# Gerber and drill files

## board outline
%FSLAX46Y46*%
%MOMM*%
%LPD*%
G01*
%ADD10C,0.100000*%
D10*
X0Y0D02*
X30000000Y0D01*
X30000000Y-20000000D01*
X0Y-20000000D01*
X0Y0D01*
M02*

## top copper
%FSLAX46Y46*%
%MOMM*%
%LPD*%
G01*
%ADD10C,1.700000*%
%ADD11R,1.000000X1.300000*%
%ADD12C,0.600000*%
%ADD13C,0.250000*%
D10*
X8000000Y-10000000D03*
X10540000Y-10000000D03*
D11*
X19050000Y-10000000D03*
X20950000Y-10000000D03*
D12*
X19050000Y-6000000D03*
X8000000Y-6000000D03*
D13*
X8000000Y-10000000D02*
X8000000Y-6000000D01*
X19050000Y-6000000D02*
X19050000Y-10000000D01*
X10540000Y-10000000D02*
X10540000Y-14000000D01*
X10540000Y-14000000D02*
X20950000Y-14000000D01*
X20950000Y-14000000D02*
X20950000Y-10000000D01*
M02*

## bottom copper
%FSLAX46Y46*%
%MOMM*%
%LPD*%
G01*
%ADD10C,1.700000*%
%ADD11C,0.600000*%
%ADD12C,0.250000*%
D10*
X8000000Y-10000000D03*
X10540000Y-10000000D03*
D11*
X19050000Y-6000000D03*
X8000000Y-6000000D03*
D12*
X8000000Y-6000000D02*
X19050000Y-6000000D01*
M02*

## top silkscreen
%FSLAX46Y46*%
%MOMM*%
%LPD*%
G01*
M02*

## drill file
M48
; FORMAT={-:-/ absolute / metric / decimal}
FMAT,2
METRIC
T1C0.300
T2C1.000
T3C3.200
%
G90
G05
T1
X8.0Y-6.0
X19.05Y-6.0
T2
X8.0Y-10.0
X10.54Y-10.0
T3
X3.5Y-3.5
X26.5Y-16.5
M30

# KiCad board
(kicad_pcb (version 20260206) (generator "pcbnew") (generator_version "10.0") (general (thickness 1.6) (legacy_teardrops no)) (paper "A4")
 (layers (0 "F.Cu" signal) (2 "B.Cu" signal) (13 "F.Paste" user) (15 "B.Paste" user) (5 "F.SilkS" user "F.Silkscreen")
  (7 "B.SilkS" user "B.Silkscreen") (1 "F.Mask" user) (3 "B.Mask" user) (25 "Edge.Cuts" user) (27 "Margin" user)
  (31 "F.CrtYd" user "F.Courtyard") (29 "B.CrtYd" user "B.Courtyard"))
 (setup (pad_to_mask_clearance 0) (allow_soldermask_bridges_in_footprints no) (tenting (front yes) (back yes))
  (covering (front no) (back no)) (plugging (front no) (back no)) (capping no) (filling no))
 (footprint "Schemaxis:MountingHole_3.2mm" (layer "F.Cu") (at 26.5 16.5)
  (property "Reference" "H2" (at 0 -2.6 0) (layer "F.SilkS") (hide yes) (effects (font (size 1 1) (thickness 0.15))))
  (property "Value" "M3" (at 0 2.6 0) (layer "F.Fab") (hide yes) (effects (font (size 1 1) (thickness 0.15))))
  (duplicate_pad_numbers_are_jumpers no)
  (pad "" np_thru_hole circle (at 0 0) (size 3.2 3.2) (drill 3.2) (layers "*.Cu" "*.Mask")))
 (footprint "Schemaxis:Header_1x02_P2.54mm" (layer "F.Cu") (at 8 10 90)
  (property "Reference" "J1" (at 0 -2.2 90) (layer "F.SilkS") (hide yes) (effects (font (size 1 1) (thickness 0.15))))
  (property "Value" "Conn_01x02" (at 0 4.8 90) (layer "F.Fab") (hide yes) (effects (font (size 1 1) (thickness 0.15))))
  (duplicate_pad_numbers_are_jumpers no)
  (pad "1" thru_hole circle (at 0 0 90) (size 1.7 1.7) (drill 1) (layers "*.Cu" "*.Mask") (remove_unused_layers no) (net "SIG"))
  (pad "2" thru_hole circle (at 0 2.54 90) (size 1.7 1.7) (drill 1) (layers "*.Cu" "*.Mask") (remove_unused_layers no) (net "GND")))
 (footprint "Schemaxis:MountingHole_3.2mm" (layer "F.Cu") (at 3.5 3.5)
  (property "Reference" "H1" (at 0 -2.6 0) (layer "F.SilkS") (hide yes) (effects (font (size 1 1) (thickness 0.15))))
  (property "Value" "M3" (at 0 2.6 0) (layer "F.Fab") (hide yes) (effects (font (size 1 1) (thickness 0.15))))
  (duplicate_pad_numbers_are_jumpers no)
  (pad "" np_thru_hole circle (at 0 0) (size 3.2 3.2) (drill 3.2) (layers "*.Cu" "*.Mask")))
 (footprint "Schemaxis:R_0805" (layer "F.Cu") (at 20 10)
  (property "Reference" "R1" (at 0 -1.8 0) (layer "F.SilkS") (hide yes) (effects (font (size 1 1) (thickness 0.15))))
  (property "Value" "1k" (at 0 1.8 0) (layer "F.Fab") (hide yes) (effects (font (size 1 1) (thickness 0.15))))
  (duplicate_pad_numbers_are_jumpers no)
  (pad "1" smd rect (at -0.95 0) (size 1 1.3) (layers "F.Cu" "F.Mask" "F.Paste") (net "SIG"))
  (pad "2" smd rect (at 0.95 0) (size 1 1.3) (layers "F.Cu" "F.Mask" "F.Paste") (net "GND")))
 (gr_rect (start 0 0) (end 30 20) (stroke (width 0.1) (type default)) (fill no) (layer "Edge.Cuts"))
 (segment (start 8 10) (end 8 6) (width 0.25) (layer "F.Cu") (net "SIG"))
 (segment (start 19.05 6) (end 19.05 10) (width 0.25) (layer "F.Cu") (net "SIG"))
 (via (at 19.05 6) (size 0.6) (drill 0.3) (layers "F.Cu" "B.Cu") (capping no) (covering (front no) (back no))
  (plugging (front no) (back no)) (filling no) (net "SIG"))
 (via (at 8 6) (size 0.6) (drill 0.3) (layers "F.Cu" "B.Cu") (capping no) (covering (front no) (back no)) (plugging (front no) (back no))
  (filling no) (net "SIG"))
 (segment (start 8 6) (end 19.05 6) (width 0.25) (layer "B.Cu") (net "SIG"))
 (segment (start 10.54 10) (end 10.54 14) (width 0.25) (layer "F.Cu") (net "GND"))
 (segment (start 10.54 14) (end 20.95 14) (width 0.25) (layer "F.Cu") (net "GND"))
 (segment (start 20.95 14) (end 20.95 10) (width 0.25) (layer "F.Cu") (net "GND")))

